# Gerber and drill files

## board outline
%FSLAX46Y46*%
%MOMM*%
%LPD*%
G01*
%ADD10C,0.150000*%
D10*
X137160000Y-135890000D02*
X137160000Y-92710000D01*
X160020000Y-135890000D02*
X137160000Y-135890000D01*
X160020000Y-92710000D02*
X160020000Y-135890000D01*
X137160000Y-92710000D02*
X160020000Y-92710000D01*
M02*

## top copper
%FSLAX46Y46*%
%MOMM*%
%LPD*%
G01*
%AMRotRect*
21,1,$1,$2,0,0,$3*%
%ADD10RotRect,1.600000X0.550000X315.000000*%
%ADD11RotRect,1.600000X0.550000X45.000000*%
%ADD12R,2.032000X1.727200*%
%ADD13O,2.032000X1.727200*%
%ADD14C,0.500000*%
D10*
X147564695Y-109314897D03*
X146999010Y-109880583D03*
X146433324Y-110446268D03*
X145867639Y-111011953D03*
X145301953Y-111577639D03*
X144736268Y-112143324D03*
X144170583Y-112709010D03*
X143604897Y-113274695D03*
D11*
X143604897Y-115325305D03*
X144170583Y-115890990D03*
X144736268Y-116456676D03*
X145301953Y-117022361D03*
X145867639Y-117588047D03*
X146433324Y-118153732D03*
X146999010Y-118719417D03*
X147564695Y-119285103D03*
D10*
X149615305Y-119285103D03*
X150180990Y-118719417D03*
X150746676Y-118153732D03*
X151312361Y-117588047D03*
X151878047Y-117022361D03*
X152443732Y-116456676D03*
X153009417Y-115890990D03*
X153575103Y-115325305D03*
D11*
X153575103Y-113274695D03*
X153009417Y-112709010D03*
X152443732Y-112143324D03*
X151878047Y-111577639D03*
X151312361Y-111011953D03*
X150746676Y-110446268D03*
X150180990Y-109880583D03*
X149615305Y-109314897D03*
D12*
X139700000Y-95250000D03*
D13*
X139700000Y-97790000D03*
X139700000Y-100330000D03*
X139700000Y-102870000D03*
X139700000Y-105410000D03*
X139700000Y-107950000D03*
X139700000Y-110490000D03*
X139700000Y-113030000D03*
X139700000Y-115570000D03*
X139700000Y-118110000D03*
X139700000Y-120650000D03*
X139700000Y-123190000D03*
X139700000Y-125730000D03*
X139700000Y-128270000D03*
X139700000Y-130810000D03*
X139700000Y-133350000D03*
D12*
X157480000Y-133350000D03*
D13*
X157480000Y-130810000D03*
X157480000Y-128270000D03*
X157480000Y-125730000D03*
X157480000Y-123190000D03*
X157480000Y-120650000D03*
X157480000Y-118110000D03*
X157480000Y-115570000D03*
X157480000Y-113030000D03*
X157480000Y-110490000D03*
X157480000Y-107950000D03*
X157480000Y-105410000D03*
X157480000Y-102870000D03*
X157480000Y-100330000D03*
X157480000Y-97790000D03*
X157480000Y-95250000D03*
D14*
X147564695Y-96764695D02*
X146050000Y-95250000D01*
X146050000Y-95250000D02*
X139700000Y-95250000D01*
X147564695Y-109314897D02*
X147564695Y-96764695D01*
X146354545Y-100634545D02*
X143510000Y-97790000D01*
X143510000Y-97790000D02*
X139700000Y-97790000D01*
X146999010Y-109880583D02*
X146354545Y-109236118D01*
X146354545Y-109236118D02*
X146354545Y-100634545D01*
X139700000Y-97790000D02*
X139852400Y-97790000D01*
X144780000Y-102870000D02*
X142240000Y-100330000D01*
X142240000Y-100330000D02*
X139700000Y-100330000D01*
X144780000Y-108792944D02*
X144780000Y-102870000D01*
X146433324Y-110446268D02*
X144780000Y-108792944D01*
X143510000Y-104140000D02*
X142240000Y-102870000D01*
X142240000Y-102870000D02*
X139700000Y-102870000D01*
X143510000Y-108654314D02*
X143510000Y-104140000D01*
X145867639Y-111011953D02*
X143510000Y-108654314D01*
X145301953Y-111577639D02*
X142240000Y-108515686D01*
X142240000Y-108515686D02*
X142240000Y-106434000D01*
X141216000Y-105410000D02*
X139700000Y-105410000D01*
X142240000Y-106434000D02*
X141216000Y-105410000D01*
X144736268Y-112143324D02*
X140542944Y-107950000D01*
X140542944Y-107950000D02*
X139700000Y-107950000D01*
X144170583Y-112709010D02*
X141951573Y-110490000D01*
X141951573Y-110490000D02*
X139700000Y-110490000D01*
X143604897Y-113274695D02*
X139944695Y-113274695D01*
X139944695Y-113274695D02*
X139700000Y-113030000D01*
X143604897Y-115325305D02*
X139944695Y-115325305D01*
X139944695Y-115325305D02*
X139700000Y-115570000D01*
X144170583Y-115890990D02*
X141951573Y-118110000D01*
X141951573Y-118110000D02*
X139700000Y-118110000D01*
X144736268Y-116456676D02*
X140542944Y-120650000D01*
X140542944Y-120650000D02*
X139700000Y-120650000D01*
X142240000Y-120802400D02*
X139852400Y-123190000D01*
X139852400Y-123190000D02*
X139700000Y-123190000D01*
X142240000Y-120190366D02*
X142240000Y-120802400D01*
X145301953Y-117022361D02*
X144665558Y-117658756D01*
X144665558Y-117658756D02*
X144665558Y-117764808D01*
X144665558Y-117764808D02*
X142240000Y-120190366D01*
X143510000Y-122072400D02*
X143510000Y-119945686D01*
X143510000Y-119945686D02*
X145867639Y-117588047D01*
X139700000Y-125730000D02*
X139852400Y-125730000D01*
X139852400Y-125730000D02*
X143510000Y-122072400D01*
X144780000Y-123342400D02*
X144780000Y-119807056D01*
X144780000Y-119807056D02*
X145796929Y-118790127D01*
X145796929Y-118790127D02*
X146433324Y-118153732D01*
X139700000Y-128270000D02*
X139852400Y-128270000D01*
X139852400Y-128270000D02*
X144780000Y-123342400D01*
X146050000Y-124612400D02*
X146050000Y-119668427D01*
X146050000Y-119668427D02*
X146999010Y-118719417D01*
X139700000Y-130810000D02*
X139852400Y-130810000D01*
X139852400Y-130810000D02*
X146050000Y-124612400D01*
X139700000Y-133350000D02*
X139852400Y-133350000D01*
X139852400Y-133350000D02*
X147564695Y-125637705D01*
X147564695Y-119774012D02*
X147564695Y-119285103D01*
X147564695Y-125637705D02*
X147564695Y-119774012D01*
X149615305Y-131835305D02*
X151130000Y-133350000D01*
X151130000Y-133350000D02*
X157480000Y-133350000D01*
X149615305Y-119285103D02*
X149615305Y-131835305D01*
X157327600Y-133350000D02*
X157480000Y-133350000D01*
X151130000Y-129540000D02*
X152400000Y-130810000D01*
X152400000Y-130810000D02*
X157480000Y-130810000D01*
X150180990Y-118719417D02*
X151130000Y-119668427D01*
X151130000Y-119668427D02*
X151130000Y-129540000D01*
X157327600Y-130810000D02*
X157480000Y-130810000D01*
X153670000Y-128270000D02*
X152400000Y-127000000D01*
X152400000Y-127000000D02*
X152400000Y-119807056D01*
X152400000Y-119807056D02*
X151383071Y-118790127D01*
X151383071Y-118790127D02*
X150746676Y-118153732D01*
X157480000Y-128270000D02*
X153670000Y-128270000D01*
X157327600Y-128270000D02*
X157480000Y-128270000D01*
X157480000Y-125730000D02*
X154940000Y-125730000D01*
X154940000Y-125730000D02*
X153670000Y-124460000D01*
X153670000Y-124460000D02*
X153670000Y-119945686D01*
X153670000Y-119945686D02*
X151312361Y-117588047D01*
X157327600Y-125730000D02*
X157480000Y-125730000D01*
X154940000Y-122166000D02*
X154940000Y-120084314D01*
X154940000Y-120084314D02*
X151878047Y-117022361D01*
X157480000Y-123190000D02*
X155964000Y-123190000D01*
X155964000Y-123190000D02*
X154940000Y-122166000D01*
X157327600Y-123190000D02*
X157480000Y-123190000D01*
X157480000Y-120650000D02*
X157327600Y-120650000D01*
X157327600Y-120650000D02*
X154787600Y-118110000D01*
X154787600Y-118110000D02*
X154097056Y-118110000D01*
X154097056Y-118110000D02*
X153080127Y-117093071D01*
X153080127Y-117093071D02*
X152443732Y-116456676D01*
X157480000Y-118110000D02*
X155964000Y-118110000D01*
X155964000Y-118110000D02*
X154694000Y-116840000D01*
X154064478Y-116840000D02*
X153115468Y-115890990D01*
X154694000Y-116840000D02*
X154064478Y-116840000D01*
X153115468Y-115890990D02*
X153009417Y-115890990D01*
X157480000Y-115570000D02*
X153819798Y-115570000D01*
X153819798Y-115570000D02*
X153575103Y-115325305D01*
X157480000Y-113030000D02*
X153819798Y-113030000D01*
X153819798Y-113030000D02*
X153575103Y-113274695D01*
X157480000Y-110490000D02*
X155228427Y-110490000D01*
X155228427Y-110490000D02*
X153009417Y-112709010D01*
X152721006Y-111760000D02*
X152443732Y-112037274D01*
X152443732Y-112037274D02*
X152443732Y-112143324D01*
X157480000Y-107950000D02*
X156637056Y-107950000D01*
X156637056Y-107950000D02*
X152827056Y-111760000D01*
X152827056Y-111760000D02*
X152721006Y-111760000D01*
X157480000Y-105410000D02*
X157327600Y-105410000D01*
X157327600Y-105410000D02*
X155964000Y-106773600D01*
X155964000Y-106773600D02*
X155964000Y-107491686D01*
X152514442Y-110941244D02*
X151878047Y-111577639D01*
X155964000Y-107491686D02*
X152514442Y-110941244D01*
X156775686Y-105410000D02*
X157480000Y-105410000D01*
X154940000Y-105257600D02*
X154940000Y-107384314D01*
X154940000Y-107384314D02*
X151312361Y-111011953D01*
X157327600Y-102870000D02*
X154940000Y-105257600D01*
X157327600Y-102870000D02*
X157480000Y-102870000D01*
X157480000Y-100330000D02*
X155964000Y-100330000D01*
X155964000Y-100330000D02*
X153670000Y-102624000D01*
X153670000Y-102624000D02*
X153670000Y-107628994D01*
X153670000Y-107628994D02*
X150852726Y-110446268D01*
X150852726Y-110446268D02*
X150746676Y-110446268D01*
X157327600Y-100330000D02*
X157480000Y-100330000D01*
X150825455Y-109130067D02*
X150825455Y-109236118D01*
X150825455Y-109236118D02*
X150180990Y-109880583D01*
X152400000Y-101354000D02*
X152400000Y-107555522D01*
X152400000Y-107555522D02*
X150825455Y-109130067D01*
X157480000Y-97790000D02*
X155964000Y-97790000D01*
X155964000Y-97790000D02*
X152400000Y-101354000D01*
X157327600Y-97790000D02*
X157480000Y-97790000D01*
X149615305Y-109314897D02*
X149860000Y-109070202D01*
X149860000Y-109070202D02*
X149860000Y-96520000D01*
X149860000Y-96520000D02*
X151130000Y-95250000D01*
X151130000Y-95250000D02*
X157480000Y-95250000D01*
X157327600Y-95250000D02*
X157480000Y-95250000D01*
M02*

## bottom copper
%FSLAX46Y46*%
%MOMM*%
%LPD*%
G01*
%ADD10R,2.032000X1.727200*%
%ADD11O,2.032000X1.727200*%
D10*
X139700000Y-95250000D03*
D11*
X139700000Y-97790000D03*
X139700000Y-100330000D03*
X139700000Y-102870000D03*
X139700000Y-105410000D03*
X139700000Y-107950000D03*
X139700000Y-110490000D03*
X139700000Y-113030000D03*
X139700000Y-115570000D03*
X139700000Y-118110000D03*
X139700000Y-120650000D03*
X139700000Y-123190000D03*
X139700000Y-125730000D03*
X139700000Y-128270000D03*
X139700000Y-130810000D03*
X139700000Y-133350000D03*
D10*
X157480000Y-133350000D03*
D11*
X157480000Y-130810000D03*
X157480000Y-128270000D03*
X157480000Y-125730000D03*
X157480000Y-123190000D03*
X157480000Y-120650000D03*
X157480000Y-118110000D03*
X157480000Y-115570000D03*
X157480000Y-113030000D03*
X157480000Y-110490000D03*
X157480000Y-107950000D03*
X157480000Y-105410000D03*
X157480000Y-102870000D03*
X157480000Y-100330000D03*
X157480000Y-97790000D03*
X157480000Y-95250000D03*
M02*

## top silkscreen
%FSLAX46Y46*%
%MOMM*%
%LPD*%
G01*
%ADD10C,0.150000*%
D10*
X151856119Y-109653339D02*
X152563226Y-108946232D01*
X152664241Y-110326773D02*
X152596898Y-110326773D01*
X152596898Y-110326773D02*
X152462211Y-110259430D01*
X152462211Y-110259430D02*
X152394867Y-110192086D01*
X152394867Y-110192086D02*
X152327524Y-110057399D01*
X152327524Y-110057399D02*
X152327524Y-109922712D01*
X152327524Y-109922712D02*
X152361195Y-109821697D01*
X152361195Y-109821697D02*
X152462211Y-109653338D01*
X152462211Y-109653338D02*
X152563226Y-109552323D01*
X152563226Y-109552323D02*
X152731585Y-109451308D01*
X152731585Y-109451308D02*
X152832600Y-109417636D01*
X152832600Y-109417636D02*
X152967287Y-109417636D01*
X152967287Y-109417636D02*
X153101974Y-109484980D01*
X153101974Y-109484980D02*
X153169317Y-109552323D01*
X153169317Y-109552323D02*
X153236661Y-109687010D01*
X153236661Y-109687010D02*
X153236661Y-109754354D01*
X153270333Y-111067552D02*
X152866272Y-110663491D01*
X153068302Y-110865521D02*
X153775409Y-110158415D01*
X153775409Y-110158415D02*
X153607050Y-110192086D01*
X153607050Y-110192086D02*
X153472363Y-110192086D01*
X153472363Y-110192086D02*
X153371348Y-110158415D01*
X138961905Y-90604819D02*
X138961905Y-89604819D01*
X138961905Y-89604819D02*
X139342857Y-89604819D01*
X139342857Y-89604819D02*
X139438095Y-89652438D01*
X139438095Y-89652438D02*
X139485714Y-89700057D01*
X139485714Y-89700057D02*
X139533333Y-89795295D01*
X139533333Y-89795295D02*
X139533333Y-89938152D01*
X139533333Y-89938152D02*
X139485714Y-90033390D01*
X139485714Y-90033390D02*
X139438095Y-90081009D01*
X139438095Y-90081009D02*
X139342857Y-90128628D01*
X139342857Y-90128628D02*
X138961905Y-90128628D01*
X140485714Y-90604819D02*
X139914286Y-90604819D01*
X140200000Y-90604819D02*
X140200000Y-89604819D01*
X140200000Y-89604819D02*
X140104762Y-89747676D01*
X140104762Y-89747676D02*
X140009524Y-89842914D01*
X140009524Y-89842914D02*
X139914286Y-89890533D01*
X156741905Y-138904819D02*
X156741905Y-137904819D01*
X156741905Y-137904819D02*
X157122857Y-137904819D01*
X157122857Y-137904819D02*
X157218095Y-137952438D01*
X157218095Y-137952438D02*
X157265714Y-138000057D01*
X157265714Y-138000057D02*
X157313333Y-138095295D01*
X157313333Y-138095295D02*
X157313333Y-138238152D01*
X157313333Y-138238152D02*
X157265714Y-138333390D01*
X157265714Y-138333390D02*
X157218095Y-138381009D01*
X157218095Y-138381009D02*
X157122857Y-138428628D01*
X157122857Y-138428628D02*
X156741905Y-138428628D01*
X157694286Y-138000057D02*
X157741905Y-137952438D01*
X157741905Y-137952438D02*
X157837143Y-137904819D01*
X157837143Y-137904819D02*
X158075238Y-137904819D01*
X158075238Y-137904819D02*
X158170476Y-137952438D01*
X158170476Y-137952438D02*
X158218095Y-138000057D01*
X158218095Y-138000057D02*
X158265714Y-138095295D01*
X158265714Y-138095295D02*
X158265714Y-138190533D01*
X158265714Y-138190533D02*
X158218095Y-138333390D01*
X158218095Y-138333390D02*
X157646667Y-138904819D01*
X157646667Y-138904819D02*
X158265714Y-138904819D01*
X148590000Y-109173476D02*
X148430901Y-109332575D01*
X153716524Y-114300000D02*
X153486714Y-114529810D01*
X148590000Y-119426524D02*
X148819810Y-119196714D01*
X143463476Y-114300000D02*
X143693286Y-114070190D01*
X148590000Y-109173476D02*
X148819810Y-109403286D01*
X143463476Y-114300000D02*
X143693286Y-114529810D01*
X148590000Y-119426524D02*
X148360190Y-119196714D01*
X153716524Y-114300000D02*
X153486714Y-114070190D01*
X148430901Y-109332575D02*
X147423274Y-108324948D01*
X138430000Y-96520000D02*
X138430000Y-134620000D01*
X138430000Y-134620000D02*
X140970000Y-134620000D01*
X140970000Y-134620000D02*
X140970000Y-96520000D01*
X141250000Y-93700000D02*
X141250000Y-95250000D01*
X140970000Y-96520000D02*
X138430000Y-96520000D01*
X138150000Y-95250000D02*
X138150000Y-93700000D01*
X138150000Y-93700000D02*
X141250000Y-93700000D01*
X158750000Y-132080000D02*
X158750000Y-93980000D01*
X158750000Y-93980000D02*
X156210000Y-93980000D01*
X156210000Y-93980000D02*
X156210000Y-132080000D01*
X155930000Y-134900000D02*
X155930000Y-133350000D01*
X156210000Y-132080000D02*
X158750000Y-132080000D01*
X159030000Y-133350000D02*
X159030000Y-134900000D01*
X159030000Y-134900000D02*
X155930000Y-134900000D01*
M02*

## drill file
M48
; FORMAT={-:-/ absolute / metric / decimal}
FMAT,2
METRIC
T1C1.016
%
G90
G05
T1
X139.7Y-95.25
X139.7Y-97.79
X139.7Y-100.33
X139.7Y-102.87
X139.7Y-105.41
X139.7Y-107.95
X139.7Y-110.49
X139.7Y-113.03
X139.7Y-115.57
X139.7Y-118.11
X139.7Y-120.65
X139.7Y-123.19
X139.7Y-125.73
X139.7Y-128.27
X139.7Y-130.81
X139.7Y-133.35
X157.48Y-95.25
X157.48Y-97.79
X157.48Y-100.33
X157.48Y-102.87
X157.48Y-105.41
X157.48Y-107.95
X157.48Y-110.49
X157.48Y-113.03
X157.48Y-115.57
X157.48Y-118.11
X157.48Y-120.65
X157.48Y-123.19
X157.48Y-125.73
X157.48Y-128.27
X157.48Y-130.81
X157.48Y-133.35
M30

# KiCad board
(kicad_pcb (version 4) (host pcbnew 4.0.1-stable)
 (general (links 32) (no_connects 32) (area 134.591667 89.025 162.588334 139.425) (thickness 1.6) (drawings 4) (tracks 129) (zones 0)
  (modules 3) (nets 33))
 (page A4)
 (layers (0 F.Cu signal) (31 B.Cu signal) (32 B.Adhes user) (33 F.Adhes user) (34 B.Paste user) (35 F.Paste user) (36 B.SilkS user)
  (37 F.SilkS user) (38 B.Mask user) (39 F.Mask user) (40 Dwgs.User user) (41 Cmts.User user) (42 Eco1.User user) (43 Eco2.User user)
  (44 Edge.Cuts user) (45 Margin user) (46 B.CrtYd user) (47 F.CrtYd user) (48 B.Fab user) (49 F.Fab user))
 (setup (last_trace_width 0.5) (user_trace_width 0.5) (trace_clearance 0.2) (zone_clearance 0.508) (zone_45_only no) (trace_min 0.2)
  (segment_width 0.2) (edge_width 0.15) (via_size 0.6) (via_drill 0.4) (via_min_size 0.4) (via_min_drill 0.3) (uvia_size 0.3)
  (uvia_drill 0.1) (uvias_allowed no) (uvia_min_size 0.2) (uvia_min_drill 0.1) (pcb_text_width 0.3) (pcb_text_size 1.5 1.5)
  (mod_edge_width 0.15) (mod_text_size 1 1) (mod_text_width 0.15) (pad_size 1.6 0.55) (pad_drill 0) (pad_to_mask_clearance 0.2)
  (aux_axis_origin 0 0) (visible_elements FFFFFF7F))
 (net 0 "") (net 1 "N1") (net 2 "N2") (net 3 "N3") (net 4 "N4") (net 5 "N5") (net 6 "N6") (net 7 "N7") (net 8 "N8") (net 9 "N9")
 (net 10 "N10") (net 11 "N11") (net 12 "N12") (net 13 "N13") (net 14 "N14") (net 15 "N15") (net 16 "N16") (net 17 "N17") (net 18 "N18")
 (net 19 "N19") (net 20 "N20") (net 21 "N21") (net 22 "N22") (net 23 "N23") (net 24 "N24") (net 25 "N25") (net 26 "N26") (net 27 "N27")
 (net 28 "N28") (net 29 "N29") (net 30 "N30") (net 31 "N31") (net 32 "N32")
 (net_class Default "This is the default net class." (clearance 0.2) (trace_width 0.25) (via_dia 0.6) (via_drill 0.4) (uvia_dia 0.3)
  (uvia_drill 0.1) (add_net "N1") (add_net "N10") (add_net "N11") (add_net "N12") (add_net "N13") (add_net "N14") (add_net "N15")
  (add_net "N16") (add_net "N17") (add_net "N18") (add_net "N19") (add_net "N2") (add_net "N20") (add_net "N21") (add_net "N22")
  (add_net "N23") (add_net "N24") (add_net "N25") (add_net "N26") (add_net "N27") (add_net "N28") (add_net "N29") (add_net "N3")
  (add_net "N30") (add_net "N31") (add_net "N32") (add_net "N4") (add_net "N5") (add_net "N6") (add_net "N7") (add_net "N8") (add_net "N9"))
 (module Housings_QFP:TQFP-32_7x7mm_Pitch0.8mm (layer F.Cu) (at 148.59 114.3 315)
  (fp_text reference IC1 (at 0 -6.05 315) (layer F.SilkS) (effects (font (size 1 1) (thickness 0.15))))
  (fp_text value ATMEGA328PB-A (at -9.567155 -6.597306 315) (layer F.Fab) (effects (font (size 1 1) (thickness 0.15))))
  (fp_line (start -3.625 -3.625) (end -3.625 -3.4) (layer F.SilkS) (width 0.15))
  (fp_line (start 3.625 -3.625) (end 3.625 -3.3) (layer F.SilkS) (width 0.15))
  (fp_line (start 3.625 3.625) (end 3.625 3.3) (layer F.SilkS) (width 0.15))
  (fp_line (start -3.625 3.625) (end -3.625 3.3) (layer F.SilkS) (width 0.15))
  (fp_line (start -3.625 -3.625) (end -3.3 -3.625) (layer F.SilkS) (width 0.15))
  (fp_line (start -3.625 3.625) (end -3.3 3.625) (layer F.SilkS) (width 0.15))
  (fp_line (start 3.625 3.625) (end 3.3 3.625) (layer F.SilkS) (width 0.15))
  (fp_line (start 3.625 -3.625) (end 3.3 -3.625) (layer F.SilkS) (width 0.15))
  (fp_line (start -3.625 -3.4) (end -5.05 -3.4) (layer F.SilkS) (width 0.15))
  (pad 1 smd rect (at -4.25 -2.8 315) (size 1.6 0.55) (layers F.Cu F.Paste F.Mask) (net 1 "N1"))
  (pad 2 smd rect (at -4.25 -2 315) (size 1.6 0.55) (layers F.Cu F.Paste F.Mask) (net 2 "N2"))
  (pad 3 smd rect (at -4.25 -1.2 315) (size 1.6 0.55) (layers F.Cu F.Paste F.Mask) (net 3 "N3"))
  (pad 4 smd rect (at -4.25 -0.4 315) (size 1.6 0.55) (layers F.Cu F.Paste F.Mask) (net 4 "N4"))
  (pad 5 smd rect (at -4.25 0.4 315) (size 1.6 0.55) (layers F.Cu F.Paste F.Mask) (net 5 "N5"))
  (pad 6 smd rect (at -4.25 1.2 315) (size 1.6 0.55) (layers F.Cu F.Paste F.Mask) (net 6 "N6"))
  (pad 7 smd rect (at -4.25 2 315) (size 1.6 0.55) (layers F.Cu F.Paste F.Mask) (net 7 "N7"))
  (pad 8 smd rect (at -4.25 2.8 315) (size 1.6 0.55) (layers F.Cu F.Paste F.Mask) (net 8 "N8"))
  (pad 9 smd rect (at -2.8 4.25 45) (size 1.6 0.55) (layers F.Cu F.Paste F.Mask) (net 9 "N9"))
  (pad 10 smd rect (at -2 4.25 45) (size 1.6 0.55) (layers F.Cu F.Paste F.Mask) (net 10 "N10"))
  (pad 11 smd rect (at -1.2 4.25 45) (size 1.6 0.55) (layers F.Cu F.Paste F.Mask) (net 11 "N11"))
  (pad 12 smd rect (at -0.4 4.25 45) (size 1.6 0.55) (layers F.Cu F.Paste F.Mask) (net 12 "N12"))
  (pad 13 smd rect (at 0.4 4.25 45) (size 1.6 0.55) (layers F.Cu F.Paste F.Mask) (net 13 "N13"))
  (pad 14 smd rect (at 1.2 4.25 45) (size 1.6 0.55) (layers F.Cu F.Paste F.Mask) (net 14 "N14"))
  (pad 15 smd rect (at 2 4.25 45) (size 1.6 0.55) (layers F.Cu F.Paste F.Mask) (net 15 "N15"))
  (pad 16 smd rect (at 2.8 4.25 45) (size 1.6 0.55) (layers F.Cu F.Paste F.Mask) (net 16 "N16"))
  (pad 17 smd rect (at 4.25 2.8 315) (size 1.6 0.55) (layers F.Cu F.Paste F.Mask) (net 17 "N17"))
  (pad 18 smd rect (at 4.25 2 315) (size 1.6 0.55) (layers F.Cu F.Paste F.Mask) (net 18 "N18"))
  (pad 19 smd rect (at 4.25 1.2 315) (size 1.6 0.55) (layers F.Cu F.Paste F.Mask) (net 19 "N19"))
  (pad 20 smd rect (at 4.25 0.4 315) (size 1.6 0.55) (layers F.Cu F.Paste F.Mask) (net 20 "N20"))
  (pad 21 smd rect (at 4.25 -0.4 315) (size 1.6 0.55) (layers F.Cu F.Paste F.Mask) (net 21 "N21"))
  (pad 22 smd rect (at 4.25 -1.2 315) (size 1.6 0.55) (layers F.Cu F.Paste F.Mask) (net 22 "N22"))
  (pad 23 smd rect (at 4.25 -2 315) (size 1.6 0.55) (layers F.Cu F.Paste F.Mask) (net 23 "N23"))
  (pad 24 smd rect (at 4.25 -2.8 315) (size 1.6 0.55) (layers F.Cu F.Paste F.Mask) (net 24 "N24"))
  (pad 25 smd rect (at 2.8 -4.25 45) (size 1.6 0.55) (layers F.Cu F.Paste F.Mask) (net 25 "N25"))
  (pad 26 smd rect (at 2 -4.25 45) (size 1.6 0.55) (layers F.Cu F.Paste F.Mask) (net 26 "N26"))
  (pad 27 smd rect (at 1.2 -4.25 45) (size 1.6 0.55) (layers F.Cu F.Paste F.Mask) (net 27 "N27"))
  (pad 28 smd rect (at 0.4 -4.25 45) (size 1.6 0.55) (layers F.Cu F.Paste F.Mask) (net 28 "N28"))
  (pad 29 smd rect (at -0.4 -4.25 45) (size 1.6 0.55) (layers F.Cu F.Paste F.Mask) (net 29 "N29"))
  (pad 30 smd rect (at -1.2 -4.25 45) (size 1.6 0.55) (layers F.Cu F.Paste F.Mask) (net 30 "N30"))
  (pad 31 smd rect (at -2 -4.25 45) (size 1.6 0.55) (layers F.Cu F.Paste F.Mask) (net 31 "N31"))
  (pad 32 smd rect (at -2.8 -4.25 45) (size 1.6 0.55) (layers F.Cu F.Paste F.Mask) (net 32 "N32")))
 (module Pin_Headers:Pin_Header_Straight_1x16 (layer F.Cu) (at 139.7 95.25)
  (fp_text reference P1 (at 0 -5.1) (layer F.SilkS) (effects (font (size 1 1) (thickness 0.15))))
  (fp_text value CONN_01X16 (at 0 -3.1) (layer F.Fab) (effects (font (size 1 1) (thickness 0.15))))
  (fp_line (start -1.27 1.27) (end -1.27 39.37) (layer F.SilkS) (width 0.15))
  (fp_line (start -1.27 39.37) (end 1.27 39.37) (layer F.SilkS) (width 0.15))
  (fp_line (start 1.27 39.37) (end 1.27 1.27) (layer F.SilkS) (width 0.15))
  (fp_line (start 1.55 -1.55) (end 1.55 0) (layer F.SilkS) (width 0.15))
  (fp_line (start 1.27 1.27) (end -1.27 1.27) (layer F.SilkS) (width 0.15))
  (fp_line (start -1.55 0) (end -1.55 -1.55) (layer F.SilkS) (width 0.15))
  (fp_line (start -1.55 -1.55) (end 1.55 -1.55) (layer F.SilkS) (width 0.15))
  (pad 1 thru_hole rect (at 0 0) (size 2.032 1.7272) (drill 1.016) (layers *.Cu *.Mask) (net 1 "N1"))
  (pad 2 thru_hole oval (at 0 2.54) (size 2.032 1.7272) (drill 1.016) (layers *.Cu *.Mask) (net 2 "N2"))
  (pad 3 thru_hole oval (at 0 5.08) (size 2.032 1.7272) (drill 1.016) (layers *.Cu *.Mask) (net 3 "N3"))
  (pad 4 thru_hole oval (at 0 7.62) (size 2.032 1.7272) (drill 1.016) (layers *.Cu *.Mask) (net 4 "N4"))
  (pad 5 thru_hole oval (at 0 10.16) (size 2.032 1.7272) (drill 1.016) (layers *.Cu *.Mask) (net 5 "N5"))
  (pad 6 thru_hole oval (at 0 12.7) (size 2.032 1.7272) (drill 1.016) (layers *.Cu *.Mask) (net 6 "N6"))
  (pad 7 thru_hole oval (at 0 15.24) (size 2.032 1.7272) (drill 1.016) (layers *.Cu *.Mask) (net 7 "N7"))
  (pad 8 thru_hole oval (at 0 17.78) (size 2.032 1.7272) (drill 1.016) (layers *.Cu *.Mask) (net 8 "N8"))
  (pad 9 thru_hole oval (at 0 20.32) (size 2.032 1.7272) (drill 1.016) (layers *.Cu *.Mask) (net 9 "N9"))
  (pad 10 thru_hole oval (at 0 22.86) (size 2.032 1.7272) (drill 1.016) (layers *.Cu *.Mask) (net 10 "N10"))
  (pad 11 thru_hole oval (at 0 25.4) (size 2.032 1.7272) (drill 1.016) (layers *.Cu *.Mask) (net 11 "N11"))
  (pad 12 thru_hole oval (at 0 27.94) (size 2.032 1.7272) (drill 1.016) (layers *.Cu *.Mask) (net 12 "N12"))
  (pad 13 thru_hole oval (at 0 30.48) (size 2.032 1.7272) (drill 1.016) (layers *.Cu *.Mask) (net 13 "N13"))
  (pad 14 thru_hole oval (at 0 33.02) (size 2.032 1.7272) (drill 1.016) (layers *.Cu *.Mask) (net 14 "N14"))
  (pad 15 thru_hole oval (at 0 35.56) (size 2.032 1.7272) (drill 1.016) (layers *.Cu *.Mask) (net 15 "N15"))
  (pad 16 thru_hole oval (at 0 38.1) (size 2.032 1.7272) (drill 1.016) (layers *.Cu *.Mask) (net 16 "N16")))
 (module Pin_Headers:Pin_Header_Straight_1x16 (layer F.Cu) (at 157.48 133.35 180)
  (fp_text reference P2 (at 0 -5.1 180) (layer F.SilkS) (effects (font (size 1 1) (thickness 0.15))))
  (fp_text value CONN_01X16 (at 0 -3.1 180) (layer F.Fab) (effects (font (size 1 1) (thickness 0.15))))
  (fp_line (start -1.27 1.27) (end -1.27 39.37) (layer F.SilkS) (width 0.15))
  (fp_line (start -1.27 39.37) (end 1.27 39.37) (layer F.SilkS) (width 0.15))
  (fp_line (start 1.27 39.37) (end 1.27 1.27) (layer F.SilkS) (width 0.15))
  (fp_line (start 1.55 -1.55) (end 1.55 0) (layer F.SilkS) (width 0.15))
  (fp_line (start 1.27 1.27) (end -1.27 1.27) (layer F.SilkS) (width 0.15))
  (fp_line (start -1.55 0) (end -1.55 -1.55) (layer F.SilkS) (width 0.15))
  (fp_line (start -1.55 -1.55) (end 1.55 -1.55) (layer F.SilkS) (width 0.15))
  (pad 1 thru_hole rect (at 0 0 180) (size 2.032 1.7272) (drill 1.016) (layers *.Cu *.Mask) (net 17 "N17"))
  (pad 2 thru_hole oval (at 0 2.54 180) (size 2.032 1.7272) (drill 1.016) (layers *.Cu *.Mask) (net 18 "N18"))
  (pad 3 thru_hole oval (at 0 5.08 180) (size 2.032 1.7272) (drill 1.016) (layers *.Cu *.Mask) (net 19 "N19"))
  (pad 4 thru_hole oval (at 0 7.62 180) (size 2.032 1.7272) (drill 1.016) (layers *.Cu *.Mask) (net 20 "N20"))
  (pad 5 thru_hole oval (at 0 10.16 180) (size 2.032 1.7272) (drill 1.016) (layers *.Cu *.Mask) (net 21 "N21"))
  (pad 6 thru_hole oval (at 0 12.7 180) (size 2.032 1.7272) (drill 1.016) (layers *.Cu *.Mask) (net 22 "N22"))
  (pad 7 thru_hole oval (at 0 15.24 180) (size 2.032 1.7272) (drill 1.016) (layers *.Cu *.Mask) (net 23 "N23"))
  (pad 8 thru_hole oval (at 0 17.78 180) (size 2.032 1.7272) (drill 1.016) (layers *.Cu *.Mask) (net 24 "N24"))
  (pad 9 thru_hole oval (at 0 20.32 180) (size 2.032 1.7272) (drill 1.016) (layers *.Cu *.Mask) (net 25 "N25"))
  (pad 10 thru_hole oval (at 0 22.86 180) (size 2.032 1.7272) (drill 1.016) (layers *.Cu *.Mask) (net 26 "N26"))
  (pad 11 thru_hole oval (at 0 25.4 180) (size 2.032 1.7272) (drill 1.016) (layers *.Cu *.Mask) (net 27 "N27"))
  (pad 12 thru_hole oval (at 0 27.94 180) (size 2.032 1.7272) (drill 1.016) (layers *.Cu *.Mask) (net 28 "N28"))
  (pad 13 thru_hole oval (at 0 30.48 180) (size 2.032 1.7272) (drill 1.016) (layers *.Cu *.Mask) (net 29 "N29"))
  (pad 14 thru_hole oval (at 0 33.02 180) (size 2.032 1.7272) (drill 1.016) (layers *.Cu *.Mask) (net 30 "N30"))
  (pad 15 thru_hole oval (at 0 35.56 180) (size 2.032 1.7272) (drill 1.016) (layers *.Cu *.Mask) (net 31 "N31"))
  (pad 16 thru_hole oval (at 0 38.1 180) (size 2.032 1.7272) (drill 1.016) (layers *.Cu *.Mask) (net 32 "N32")))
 (gr_line (start 137.16 135.89) (end 137.16 92.71) (layer Edge.Cuts) (width 0.15))
 (gr_line (start 160.02 135.89) (end 137.16 135.89) (layer Edge.Cuts) (width 0.15))
 (gr_line (start 160.02 92.71) (end 160.02 135.89) (layer Edge.Cuts) (width 0.15))
 (gr_line (start 137.16 92.71) (end 160.02 92.71) (layer Edge.Cuts) (width 0.15))
 (segment (start 147.564695 96.764695) (end 146.05 95.25) (width 0.5) (layer F.Cu) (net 1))
 (segment (start 146.05 95.25) (end 139.7 95.25) (width 0.5) (layer F.Cu) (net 1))
 (segment (start 147.564695 109.314897) (end 147.564695 96.764695) (width 0.5) (layer F.Cu) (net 1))
 (segment (start 146.354545 100.634545) (end 143.51 97.79) (width 0.5) (layer F.Cu) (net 2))
 (segment (start 143.51 97.79) (end 139.7 97.79) (width 0.5) (layer F.Cu) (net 2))
 (segment (start 146.99901 109.880583) (end 146.354545 109.236118) (width 0.5) (layer F.Cu) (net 2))
 (segment (start 146.354545 109.236118) (end 146.354545 100.634545) (width 0.5) (layer F.Cu) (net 2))
 (segment (start 139.7 97.79) (end 139.8524 97.79) (width 0.5) (layer F.Cu) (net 2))
 (segment (start 144.78 102.87) (end 142.24 100.33) (width 0.5) (layer F.Cu) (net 3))
 (segment (start 142.24 100.33) (end 139.7 100.33) (width 0.5) (layer F.Cu) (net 3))
 (segment (start 144.78 108.792944) (end 144.78 102.87) (width 0.5) (layer F.Cu) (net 3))
 (segment (start 146.433324 110.446268) (end 144.78 108.792944) (width 0.5) (layer F.Cu) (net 3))
 (segment (start 143.51 104.14) (end 142.24 102.87) (width 0.5) (layer F.Cu) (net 4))
 (segment (start 142.24 102.87) (end 139.7 102.87) (width 0.5) (layer F.Cu) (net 4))
 (segment (start 143.51 108.654314) (end 143.51 104.14) (width 0.5) (layer F.Cu) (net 4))
 (segment (start 145.867639 111.011953) (end 143.51 108.654314) (width 0.5) (layer F.Cu) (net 4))
 (segment (start 145.301953 111.577639) (end 142.24 108.515686) (width 0.5) (layer F.Cu) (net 5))
 (segment (start 142.24 108.515686) (end 142.24 106.434) (width 0.5) (layer F.Cu) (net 5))
 (segment (start 141.216 105.41) (end 139.7 105.41) (width 0.5) (layer F.Cu) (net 5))
 (segment (start 142.24 106.434) (end 141.216 105.41) (width 0.5) (layer F.Cu) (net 5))
 (segment (start 144.736268 112.143324) (end 140.542944 107.95) (width 0.5) (layer F.Cu) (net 6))
 (segment (start 140.542944 107.95) (end 139.7 107.95) (width 0.5) (layer F.Cu) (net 6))
 (segment (start 144.170583 112.70901) (end 141.951573 110.49) (width 0.5) (layer F.Cu) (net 7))
 (segment (start 141.951573 110.49) (end 139.7 110.49) (width 0.5) (layer F.Cu) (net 7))
 (segment (start 143.604897 113.274695) (end 139.944695 113.274695) (width 0.5) (layer F.Cu) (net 8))
 (segment (start 139.944695 113.274695) (end 139.7 113.03) (width 0.5) (layer F.Cu) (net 8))
 (segment (start 143.604897 115.325305) (end 139.944695 115.325305) (width 0.5) (layer F.Cu) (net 9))
 (segment (start 139.944695 115.325305) (end 139.7 115.57) (width 0.5) (layer F.Cu) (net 9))
 (segment (start 144.170583 115.89099) (end 141.951573 118.11) (width 0.5) (layer F.Cu) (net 10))
 (segment (start 141.951573 118.11) (end 139.7 118.11) (width 0.5) (layer F.Cu) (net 10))
 (segment (start 144.736268 116.456676) (end 140.542944 120.65) (width 0.5) (layer F.Cu) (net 11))
 (segment (start 140.542944 120.65) (end 139.7 120.65) (width 0.5) (layer F.Cu) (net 11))
 (segment (start 142.24 120.8024) (end 139.8524 123.19) (width 0.5) (layer F.Cu) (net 12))
 (segment (start 139.8524 123.19) (end 139.7 123.19) (width 0.5) (layer F.Cu) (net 12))
 (segment (start 142.24 120.190366) (end 142.24 120.8024) (width 0.5) (layer F.Cu) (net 12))
 (segment (start 145.301953 117.022361) (end 144.665558 117.658756) (width 0.5) (layer F.Cu) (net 12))
 (segment (start 144.665558 117.658756) (end 144.665558 117.764808) (width 0.5) (layer F.Cu) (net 12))
 (segment (start 144.665558 117.764808) (end 142.24 120.190366) (width 0.5) (layer F.Cu) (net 12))
 (segment (start 143.51 122.0724) (end 143.51 119.945686) (width 0.5) (layer F.Cu) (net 13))
 (segment (start 143.51 119.945686) (end 145.867639 117.588047) (width 0.5) (layer F.Cu) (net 13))
 (segment (start 139.7 125.73) (end 139.8524 125.73) (width 0.5) (layer F.Cu) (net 13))
 (segment (start 139.8524 125.73) (end 143.51 122.0724) (width 0.5) (layer F.Cu) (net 13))
 (segment (start 144.78 123.3424) (end 144.78 119.807056) (width 0.5) (layer F.Cu) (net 14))
 (segment (start 144.78 119.807056) (end 145.796929 118.790127) (width 0.5) (layer F.Cu) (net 14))
 (segment (start 145.796929 118.790127) (end 146.433324 118.153732) (width 0.5) (layer F.Cu) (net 14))
 (segment (start 139.7 128.27) (end 139.8524 128.27) (width 0.5) (layer F.Cu) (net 14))
 (segment (start 139.8524 128.27) (end 144.78 123.3424) (width 0.5) (layer F.Cu) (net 14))
 (segment (start 146.05 124.6124) (end 146.05 119.668427) (width 0.5) (layer F.Cu) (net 15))
 (segment (start 146.05 119.668427) (end 146.99901 118.719417) (width 0.5) (layer F.Cu) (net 15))
 (segment (start 139.7 130.81) (end 139.8524 130.81) (width 0.5) (layer F.Cu) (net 15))
 (segment (start 139.8524 130.81) (end 146.05 124.6124) (width 0.5) (layer F.Cu) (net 15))
 (segment (start 139.7 133.35) (end 139.8524 133.35) (width 0.5) (layer F.Cu) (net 16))
 (segment (start 139.8524 133.35) (end 147.564695 125.637705) (width 0.5) (layer F.Cu) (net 16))
 (segment (start 147.564695 119.774012) (end 147.564695 119.285103) (width 0.5) (layer F.Cu) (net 16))
 (segment (start 147.564695 125.637705) (end 147.564695 119.774012) (width 0.5) (layer F.Cu) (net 16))
 (segment (start 149.615305 131.835305) (end 151.13 133.35) (width 0.5) (layer F.Cu) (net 17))
 (segment (start 151.13 133.35) (end 157.48 133.35) (width 0.5) (layer F.Cu) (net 17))
 (segment (start 149.615305 119.285103) (end 149.615305 131.835305) (width 0.5) (layer F.Cu) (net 17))
 (segment (start 157.3276 133.35) (end 157.48 133.35) (width 0.5) (layer F.Cu) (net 17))
 (segment (start 151.13 129.54) (end 152.4 130.81) (width 0.5) (layer F.Cu) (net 18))
 (segment (start 152.4 130.81) (end 157.48 130.81) (width 0.5) (layer F.Cu) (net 18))
 (segment (start 150.18099 118.719417) (end 151.13 119.668427) (width 0.5) (layer F.Cu) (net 18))
 (segment (start 151.13 119.668427) (end 151.13 129.54) (width 0.5) (layer F.Cu) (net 18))
 (segment (start 157.3276 130.81) (end 157.48 130.81) (width 0.5) (layer F.Cu) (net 18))
 (segment (start 153.67 128.27) (end 152.4 127) (width 0.5) (layer F.Cu) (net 19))
 (segment (start 152.4 127) (end 152.4 119.807056) (width 0.5) (layer F.Cu) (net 19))
 (segment (start 152.4 119.807056) (end 151.383071 118.790127) (width 0.5) (layer F.Cu) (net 19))
 (segment (start 151.383071 118.790127) (end 150.746676 118.153732) (width 0.5) (layer F.Cu) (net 19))
 (segment (start 157.48 128.27) (end 153.67 128.27) (width 0.5) (layer F.Cu) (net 19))
 (segment (start 157.3276 128.27) (end 157.48 128.27) (width 0.5) (layer F.Cu) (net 19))
 (segment (start 157.48 125.73) (end 154.94 125.73) (width 0.5) (layer F.Cu) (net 20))
 (segment (start 154.94 125.73) (end 153.67 124.46) (width 0.5) (layer F.Cu) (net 20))
 (segment (start 153.67 124.46) (end 153.67 119.945686) (width 0.5) (layer F.Cu) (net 20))
 (segment (start 153.67 119.945686) (end 151.312361 117.588047) (width 0.5) (layer F.Cu) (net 20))
 (segment (start 157.3276 125.73) (end 157.48 125.73) (width 0.5) (layer F.Cu) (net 20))
 (segment (start 154.94 122.166) (end 154.94 120.084314) (width 0.5) (layer F.Cu) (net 21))
 (segment (start 154.94 120.084314) (end 151.878047 117.022361) (width 0.5) (layer F.Cu) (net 21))
 (segment (start 157.48 123.19) (end 155.964 123.19) (width 0.5) (layer F.Cu) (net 21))
 (segment (start 155.964 123.19) (end 154.94 122.166) (width 0.5) (layer F.Cu) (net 21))
 (segment (start 157.3276 123.19) (end 157.48 123.19) (width 0.5) (layer F.Cu) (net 21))
 (segment (start 157.48 120.65) (end 157.3276 120.65) (width 0.5) (layer F.Cu) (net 22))
 (segment (start 157.3276 120.65) (end 154.7876 118.11) (width 0.5) (layer F.Cu) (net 22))
 (segment (start 154.7876 118.11) (end 154.097056 118.11) (width 0.5) (layer F.Cu) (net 22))
 (segment (start 154.097056 118.11) (end 153.080127 117.093071) (width 0.5) (layer F.Cu) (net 22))
 (segment (start 153.080127 117.093071) (end 152.443732 116.456676) (width 0.5) (layer F.Cu) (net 22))
 (segment (start 157.48 118.11) (end 155.964 118.11) (width 0.5) (layer F.Cu) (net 23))
 (segment (start 155.964 118.11) (end 154.694 116.84) (width 0.5) (layer F.Cu) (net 23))
 (segment (start 154.064478 116.84) (end 153.115468 115.89099) (width 0.5) (layer F.Cu) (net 23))
 (segment (start 154.694 116.84) (end 154.064478 116.84) (width 0.5) (layer F.Cu) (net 23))
 (segment (start 153.115468 115.89099) (end 153.009417 115.89099) (width 0.5) (layer F.Cu) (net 23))
 (segment (start 157.48 115.57) (end 153.819798 115.57) (width 0.5) (layer F.Cu) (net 24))
 (segment (start 153.819798 115.57) (end 153.575103 115.325305) (width 0.5) (layer F.Cu) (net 24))
 (segment (start 157.48 113.03) (end 153.819798 113.03) (width 0.5) (layer F.Cu) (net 25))
 (segment (start 153.819798 113.03) (end 153.575103 113.274695) (width 0.5) (layer F.Cu) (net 25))
 (segment (start 157.48 110.49) (end 155.228427 110.49) (width 0.5) (layer F.Cu) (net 26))
 (segment (start 155.228427 110.49) (end 153.009417 112.70901) (width 0.5) (layer F.Cu) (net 26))
 (segment (start 152.721006 111.76) (end 152.443732 112.037274) (width 0.5) (layer F.Cu) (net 27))
 (segment (start 152.443732 112.037274) (end 152.443732 112.143324) (width 0.5) (layer F.Cu) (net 27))
 (segment (start 157.48 107.95) (end 156.637056 107.95) (width 0.5) (layer F.Cu) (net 27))
 (segment (start 156.637056 107.95) (end 152.827056 111.76) (width 0.5) (layer F.Cu) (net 27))
 (segment (start 152.827056 111.76) (end 152.721006 111.76) (width 0.5) (layer F.Cu) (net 27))
 (segment (start 157.48 105.41) (end 157.3276 105.41) (width 0.5) (layer F.Cu) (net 28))
 (segment (start 157.3276 105.41) (end 155.964 106.7736) (width 0.5) (layer F.Cu) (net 28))
 (segment (start 155.964 106.7736) (end 155.964 107.491686) (width 0.5) (layer F.Cu) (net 28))
 (segment (start 152.514442 110.941244) (end 151.878047 111.577639) (width 0.5) (layer F.Cu) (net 28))
 (segment (start 155.964 107.491686) (end 152.514442 110.941244) (width 0.5) (layer F.Cu) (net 28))
 (segment (start 156.775686 105.41) (end 157.48 105.41) (width 0.5) (layer F.Cu) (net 28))
 (segment (start 154.94 105.2576) (end 154.94 107.384314) (width 0.5) (layer F.Cu) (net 29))
 (segment (start 154.94 107.384314) (end 151.312361 111.011953) (width 0.5) (layer F.Cu) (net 29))
 (segment (start 157.3276 102.87) (end 154.94 105.2576) (width 0.5) (layer F.Cu) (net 29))
 (segment (start 157.3276 102.87) (end 157.48 102.87) (width 0.5) (layer F.Cu) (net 29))
 (segment (start 157.48 100.33) (end 155.964 100.33) (width 0.5) (layer F.Cu) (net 30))
 (segment (start 155.964 100.33) (end 153.67 102.624) (width 0.5) (layer F.Cu) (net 30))
 (segment (start 153.67 102.624) (end 153.67 107.628994) (width 0.5) (layer F.Cu) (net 30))
 (segment (start 153.67 107.628994) (end 150.852726 110.446268) (width 0.5) (layer F.Cu) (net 30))
 (segment (start 150.852726 110.446268) (end 150.746676 110.446268) (width 0.5) (layer F.Cu) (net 30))
 (segment (start 157.3276 100.33) (end 157.48 100.33) (width 0.5) (layer F.Cu) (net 30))
 (segment (start 150.825455 109.130067) (end 150.825455 109.236118) (width 0.5) (layer F.Cu) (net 31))
 (segment (start 150.825455 109.236118) (end 150.18099 109.880583) (width 0.5) (layer F.Cu) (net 31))
 (segment (start 152.4 101.354) (end 152.4 107.555522) (width 0.5) (layer F.Cu) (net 31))
 (segment (start 152.4 107.555522) (end 150.825455 109.130067) (width 0.5) (layer F.Cu) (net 31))
 (segment (start 157.48 97.79) (end 155.964 97.79) (width 0.5) (layer F.Cu) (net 31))
 (segment (start 155.964 97.79) (end 152.4 101.354) (width 0.5) (layer F.Cu) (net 31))
 (segment (start 157.3276 97.79) (end 157.48 97.79) (width 0.5) (layer F.Cu) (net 31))
 (segment (start 149.615305 109.314897) (end 149.86 109.070202) (width 0.5) (layer F.Cu) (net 32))
 (segment (start 149.86 109.070202) (end 149.86 96.52) (width 0.5) (layer F.Cu) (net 32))
 (segment (start 149.86 96.52) (end 151.13 95.25) (width 0.5) (layer F.Cu) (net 32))
 (segment (start 151.13 95.25) (end 157.48 95.25) (width 0.5) (layer F.Cu) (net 32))
 (segment (start 157.3276 95.25) (end 157.48 95.25) (width 0.5) (layer F.Cu) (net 32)))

